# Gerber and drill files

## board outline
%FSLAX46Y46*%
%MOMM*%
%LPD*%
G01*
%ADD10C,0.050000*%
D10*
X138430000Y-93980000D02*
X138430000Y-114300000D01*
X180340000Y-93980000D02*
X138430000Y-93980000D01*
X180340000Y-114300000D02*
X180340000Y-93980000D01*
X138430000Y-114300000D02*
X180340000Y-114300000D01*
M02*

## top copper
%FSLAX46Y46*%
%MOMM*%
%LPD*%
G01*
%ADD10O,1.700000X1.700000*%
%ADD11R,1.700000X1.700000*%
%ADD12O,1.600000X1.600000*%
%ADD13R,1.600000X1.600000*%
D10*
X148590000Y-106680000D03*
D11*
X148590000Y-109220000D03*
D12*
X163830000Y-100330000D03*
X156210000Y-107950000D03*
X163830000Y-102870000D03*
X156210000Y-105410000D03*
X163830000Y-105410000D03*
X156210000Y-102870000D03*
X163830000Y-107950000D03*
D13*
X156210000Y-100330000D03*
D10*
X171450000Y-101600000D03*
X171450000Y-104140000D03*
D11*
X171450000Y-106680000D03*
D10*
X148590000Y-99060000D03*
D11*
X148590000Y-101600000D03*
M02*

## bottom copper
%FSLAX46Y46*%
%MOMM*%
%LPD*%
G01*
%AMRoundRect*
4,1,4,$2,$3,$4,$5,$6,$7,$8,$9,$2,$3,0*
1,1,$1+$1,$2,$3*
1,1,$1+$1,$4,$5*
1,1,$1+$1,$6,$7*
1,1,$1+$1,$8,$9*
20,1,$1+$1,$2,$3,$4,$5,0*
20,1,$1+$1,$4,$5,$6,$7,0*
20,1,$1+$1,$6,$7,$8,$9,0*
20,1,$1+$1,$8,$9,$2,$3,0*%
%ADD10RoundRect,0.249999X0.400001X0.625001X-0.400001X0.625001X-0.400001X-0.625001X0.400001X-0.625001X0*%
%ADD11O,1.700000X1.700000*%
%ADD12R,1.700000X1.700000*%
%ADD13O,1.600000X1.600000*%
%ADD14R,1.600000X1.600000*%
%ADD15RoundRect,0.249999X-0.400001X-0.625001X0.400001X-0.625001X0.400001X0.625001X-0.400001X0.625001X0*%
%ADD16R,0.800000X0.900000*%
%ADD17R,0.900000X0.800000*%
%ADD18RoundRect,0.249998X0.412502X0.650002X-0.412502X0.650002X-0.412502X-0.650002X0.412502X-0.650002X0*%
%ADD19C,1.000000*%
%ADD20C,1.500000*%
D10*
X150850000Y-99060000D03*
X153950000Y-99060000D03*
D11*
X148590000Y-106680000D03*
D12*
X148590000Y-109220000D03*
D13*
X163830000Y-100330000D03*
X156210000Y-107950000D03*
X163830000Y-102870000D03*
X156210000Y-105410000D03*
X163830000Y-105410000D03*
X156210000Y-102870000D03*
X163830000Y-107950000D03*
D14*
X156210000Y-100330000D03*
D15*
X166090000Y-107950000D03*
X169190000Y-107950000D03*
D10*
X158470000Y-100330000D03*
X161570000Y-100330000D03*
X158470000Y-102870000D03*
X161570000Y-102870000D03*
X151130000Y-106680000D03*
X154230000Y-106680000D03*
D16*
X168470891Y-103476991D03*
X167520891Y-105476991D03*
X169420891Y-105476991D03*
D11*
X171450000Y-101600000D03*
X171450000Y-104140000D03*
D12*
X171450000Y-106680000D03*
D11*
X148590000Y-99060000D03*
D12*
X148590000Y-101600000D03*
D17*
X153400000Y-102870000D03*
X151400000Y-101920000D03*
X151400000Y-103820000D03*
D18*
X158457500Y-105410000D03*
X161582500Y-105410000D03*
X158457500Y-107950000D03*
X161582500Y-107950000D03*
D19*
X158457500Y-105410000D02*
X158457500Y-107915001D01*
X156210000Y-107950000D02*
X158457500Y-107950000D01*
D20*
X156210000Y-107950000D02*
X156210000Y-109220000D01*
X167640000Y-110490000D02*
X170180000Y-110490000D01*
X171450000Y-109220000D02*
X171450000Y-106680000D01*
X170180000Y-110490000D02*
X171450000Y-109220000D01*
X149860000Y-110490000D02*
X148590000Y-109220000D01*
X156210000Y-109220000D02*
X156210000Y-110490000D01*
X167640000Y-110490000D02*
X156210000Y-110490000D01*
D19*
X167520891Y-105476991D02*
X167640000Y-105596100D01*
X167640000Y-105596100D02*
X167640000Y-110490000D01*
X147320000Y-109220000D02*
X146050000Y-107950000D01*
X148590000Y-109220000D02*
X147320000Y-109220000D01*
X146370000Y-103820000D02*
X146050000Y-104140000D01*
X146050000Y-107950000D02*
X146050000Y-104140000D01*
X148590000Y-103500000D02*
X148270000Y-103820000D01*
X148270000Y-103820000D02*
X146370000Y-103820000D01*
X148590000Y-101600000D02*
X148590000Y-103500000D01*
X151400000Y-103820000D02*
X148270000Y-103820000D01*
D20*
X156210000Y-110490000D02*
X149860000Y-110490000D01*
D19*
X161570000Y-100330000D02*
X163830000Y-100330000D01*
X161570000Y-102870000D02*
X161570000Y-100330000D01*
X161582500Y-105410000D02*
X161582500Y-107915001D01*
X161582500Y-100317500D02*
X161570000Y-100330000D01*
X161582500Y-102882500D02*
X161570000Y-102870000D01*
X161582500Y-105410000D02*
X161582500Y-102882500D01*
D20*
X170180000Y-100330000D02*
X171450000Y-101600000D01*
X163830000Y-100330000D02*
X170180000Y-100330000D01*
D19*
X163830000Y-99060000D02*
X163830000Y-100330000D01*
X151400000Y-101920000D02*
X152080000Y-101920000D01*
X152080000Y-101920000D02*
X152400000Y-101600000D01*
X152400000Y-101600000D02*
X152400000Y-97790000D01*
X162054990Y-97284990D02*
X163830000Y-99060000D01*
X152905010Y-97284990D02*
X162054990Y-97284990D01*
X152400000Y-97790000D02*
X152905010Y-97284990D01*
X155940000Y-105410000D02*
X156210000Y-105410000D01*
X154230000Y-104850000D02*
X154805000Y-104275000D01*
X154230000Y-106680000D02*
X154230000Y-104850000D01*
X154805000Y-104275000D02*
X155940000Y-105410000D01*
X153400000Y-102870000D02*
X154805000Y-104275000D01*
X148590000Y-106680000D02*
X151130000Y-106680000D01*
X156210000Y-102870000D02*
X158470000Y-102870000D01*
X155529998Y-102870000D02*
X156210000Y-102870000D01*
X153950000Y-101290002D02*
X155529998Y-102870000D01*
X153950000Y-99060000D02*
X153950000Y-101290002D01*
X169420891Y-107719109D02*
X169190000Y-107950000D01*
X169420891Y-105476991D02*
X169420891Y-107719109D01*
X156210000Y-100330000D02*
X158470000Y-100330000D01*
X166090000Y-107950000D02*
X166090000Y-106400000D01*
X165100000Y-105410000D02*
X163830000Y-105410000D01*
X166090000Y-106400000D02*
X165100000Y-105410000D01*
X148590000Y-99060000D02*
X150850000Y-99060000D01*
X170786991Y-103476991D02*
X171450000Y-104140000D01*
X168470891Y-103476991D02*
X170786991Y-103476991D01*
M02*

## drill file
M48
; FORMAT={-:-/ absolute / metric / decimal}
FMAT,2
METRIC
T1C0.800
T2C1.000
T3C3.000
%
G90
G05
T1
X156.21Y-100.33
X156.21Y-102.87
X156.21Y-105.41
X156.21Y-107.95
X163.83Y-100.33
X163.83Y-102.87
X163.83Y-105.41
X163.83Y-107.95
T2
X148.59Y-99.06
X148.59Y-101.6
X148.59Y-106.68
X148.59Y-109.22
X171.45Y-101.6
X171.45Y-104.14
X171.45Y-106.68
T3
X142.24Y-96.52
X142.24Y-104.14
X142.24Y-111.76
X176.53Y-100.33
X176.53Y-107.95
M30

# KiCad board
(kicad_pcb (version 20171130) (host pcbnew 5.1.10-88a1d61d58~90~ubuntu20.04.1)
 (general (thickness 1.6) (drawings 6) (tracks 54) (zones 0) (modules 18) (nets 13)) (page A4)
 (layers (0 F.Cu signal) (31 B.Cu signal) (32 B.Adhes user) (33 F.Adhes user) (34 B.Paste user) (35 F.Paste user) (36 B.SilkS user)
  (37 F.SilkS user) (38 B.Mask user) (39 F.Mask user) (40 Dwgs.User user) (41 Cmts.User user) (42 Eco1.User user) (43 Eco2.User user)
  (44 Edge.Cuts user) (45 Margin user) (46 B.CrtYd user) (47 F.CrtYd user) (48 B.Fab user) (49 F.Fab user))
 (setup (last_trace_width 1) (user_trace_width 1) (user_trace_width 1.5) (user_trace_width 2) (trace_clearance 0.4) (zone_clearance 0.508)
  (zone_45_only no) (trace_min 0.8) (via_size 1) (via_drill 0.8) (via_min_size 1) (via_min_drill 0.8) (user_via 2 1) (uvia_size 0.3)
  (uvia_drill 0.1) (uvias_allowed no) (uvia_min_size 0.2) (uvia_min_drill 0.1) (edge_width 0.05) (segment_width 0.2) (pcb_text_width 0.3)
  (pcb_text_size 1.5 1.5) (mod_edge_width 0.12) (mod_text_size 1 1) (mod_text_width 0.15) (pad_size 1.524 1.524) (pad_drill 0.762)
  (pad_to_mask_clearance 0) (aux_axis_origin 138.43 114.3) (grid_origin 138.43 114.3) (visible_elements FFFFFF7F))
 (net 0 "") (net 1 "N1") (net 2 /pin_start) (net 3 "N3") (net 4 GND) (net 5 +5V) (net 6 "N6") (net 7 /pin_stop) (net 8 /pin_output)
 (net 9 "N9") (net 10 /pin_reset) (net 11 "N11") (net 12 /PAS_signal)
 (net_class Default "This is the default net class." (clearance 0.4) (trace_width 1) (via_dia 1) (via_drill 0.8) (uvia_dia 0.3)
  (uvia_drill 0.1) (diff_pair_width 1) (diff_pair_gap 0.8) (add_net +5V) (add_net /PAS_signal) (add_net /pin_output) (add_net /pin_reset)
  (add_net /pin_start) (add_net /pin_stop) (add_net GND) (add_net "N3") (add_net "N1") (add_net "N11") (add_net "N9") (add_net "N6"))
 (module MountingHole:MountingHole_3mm (layer F.Cu) (at 176.53 107.95)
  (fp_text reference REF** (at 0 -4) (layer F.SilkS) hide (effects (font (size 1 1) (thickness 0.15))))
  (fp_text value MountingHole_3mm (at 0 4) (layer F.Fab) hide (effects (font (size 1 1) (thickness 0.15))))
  (pad 1 np_thru_hole circle (at 0 0) (size 3 3) (drill 3) (layers *.Cu *.Mask)))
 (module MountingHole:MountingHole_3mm (layer F.Cu) (at 176.53 100.33)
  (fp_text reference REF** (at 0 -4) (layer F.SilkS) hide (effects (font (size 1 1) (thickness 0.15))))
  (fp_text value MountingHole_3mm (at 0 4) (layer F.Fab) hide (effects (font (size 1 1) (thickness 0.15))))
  (pad 1 np_thru_hole circle (at 0 0) (size 3 3) (drill 3) (layers *.Cu *.Mask)))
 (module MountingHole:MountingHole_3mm (layer F.Cu) (at 142.24 104.14)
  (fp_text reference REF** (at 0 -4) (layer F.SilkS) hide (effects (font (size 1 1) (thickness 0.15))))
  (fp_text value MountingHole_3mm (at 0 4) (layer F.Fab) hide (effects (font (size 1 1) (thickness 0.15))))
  (pad 1 np_thru_hole circle (at 0 0) (size 3 3) (drill 3) (layers *.Cu *.Mask)))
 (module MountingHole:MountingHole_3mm (layer F.Cu) (at 142.24 111.76)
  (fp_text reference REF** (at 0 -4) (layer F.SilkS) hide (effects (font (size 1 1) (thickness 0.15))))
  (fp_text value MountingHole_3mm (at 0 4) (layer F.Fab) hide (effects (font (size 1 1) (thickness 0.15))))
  (pad 1 np_thru_hole circle (at 0 0) (size 3 3) (drill 3) (layers *.Cu *.Mask)))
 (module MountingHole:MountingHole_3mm (layer F.Cu) (at 142.24 96.52)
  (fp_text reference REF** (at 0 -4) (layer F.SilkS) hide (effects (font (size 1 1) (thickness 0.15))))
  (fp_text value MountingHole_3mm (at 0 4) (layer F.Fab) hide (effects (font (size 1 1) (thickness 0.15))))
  (pad 1 np_thru_hole circle (at 0 0) (size 3 3) (drill 3) (layers *.Cu *.Mask)))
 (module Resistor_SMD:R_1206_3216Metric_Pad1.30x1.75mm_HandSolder (layer B.Cu) (at 152.4 99.06 180)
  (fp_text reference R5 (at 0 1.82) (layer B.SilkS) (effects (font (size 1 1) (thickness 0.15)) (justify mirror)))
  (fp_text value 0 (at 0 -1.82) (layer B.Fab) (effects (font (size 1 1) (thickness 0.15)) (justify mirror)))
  (pad 2 smd roundrect (at 1.55 0 180) (size 1.3 1.75) (layers B.Cu B.Paste B.Mask) (roundrect_rratio 0.1923069230769231) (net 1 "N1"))
  (pad 1 smd roundrect (at -1.55 0 180) (size 1.3 1.75) (layers B.Cu B.Paste B.Mask) (roundrect_rratio 0.1923069230769231)
   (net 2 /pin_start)))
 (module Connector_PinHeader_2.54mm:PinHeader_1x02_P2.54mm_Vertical (layer F.Cu) (at 148.59 109.22 180)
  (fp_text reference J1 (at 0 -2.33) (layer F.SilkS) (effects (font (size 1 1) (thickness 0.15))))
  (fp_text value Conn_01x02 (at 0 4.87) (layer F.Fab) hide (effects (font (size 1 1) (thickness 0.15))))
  (pad 2 thru_hole oval (at 0 2.54 180) (size 1.7 1.7) (drill 1) (layers *.Cu *.Mask) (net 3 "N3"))
  (pad 1 thru_hole rect (at 0 0 180) (size 1.7 1.7) (drill 1) (layers *.Cu *.Mask) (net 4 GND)))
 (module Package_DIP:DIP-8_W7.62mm (layer F.Cu) (at 156.21 100.33)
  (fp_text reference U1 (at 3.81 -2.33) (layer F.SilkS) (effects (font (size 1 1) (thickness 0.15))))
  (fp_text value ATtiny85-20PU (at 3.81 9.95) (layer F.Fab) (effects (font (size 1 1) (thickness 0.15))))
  (pad 8 thru_hole oval (at 7.62 0) (size 1.6 1.6) (drill 0.8) (layers *.Cu *.Mask) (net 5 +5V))
  (pad 4 thru_hole oval (at 0 7.62) (size 1.6 1.6) (drill 0.8) (layers *.Cu *.Mask) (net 4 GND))
  (pad 7 thru_hole oval (at 7.62 2.54) (size 1.6 1.6) (drill 0.8) (layers *.Cu *.Mask) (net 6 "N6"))
  (pad 3 thru_hole oval (at 0 5.08) (size 1.6 1.6) (drill 0.8) (layers *.Cu *.Mask) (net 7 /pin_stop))
  (pad 6 thru_hole oval (at 7.62 5.08) (size 1.6 1.6) (drill 0.8) (layers *.Cu *.Mask) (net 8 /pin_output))
  (pad 2 thru_hole oval (at 0 2.54) (size 1.6 1.6) (drill 0.8) (layers *.Cu *.Mask) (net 2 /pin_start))
  (pad 5 thru_hole oval (at 7.62 7.62) (size 1.6 1.6) (drill 0.8) (layers *.Cu *.Mask) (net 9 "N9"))
  (pad 1 thru_hole rect (at 0 0) (size 1.6 1.6) (drill 0.8) (layers *.Cu *.Mask) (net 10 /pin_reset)))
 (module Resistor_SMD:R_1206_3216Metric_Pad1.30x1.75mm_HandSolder (layer B.Cu) (at 167.64 107.95)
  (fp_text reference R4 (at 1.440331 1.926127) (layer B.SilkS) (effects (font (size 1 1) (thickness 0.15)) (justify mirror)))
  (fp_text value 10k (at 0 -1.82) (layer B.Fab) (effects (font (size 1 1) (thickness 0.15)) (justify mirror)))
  (pad 1 smd roundrect (at -1.55 0) (size 1.3 1.75) (layers B.Cu B.Paste B.Mask) (roundrect_rratio 0.1923069230769231) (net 8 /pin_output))
  (pad 2 smd roundrect (at 1.55 0) (size 1.3 1.75) (layers B.Cu B.Paste B.Mask) (roundrect_rratio 0.1923069230769231) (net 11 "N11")))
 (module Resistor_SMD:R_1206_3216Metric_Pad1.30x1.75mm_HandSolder (layer B.Cu) (at 160.02 100.33 180)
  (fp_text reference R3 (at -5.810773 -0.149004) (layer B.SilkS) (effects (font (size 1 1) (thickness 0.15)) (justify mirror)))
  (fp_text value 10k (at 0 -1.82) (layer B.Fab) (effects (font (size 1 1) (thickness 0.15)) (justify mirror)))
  (pad 2 smd roundrect (at 1.55 0 180) (size 1.3 1.75) (layers B.Cu B.Paste B.Mask) (roundrect_rratio 0.1923069230769231)
   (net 10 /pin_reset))
  (pad 1 smd roundrect (at -1.55 0 180) (size 1.3 1.75) (layers B.Cu B.Paste B.Mask) (roundrect_rratio 0.1923069230769231) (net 5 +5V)))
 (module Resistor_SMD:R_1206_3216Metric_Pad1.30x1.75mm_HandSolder (layer B.Cu) (at 160.02 102.87 180)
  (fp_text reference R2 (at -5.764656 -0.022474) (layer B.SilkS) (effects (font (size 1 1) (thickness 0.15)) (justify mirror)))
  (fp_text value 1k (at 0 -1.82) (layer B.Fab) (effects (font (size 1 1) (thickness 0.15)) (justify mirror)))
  (pad 2 smd roundrect (at 1.55 0 180) (size 1.3 1.75) (layers B.Cu B.Paste B.Mask) (roundrect_rratio 0.1923069230769231) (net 2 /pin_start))
  (pad 1 smd roundrect (at -1.55 0 180) (size 1.3 1.75) (layers B.Cu B.Paste B.Mask) (roundrect_rratio 0.1923069230769231) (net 5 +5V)))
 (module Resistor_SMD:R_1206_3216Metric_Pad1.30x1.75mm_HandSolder (layer B.Cu) (at 152.68 106.68 180)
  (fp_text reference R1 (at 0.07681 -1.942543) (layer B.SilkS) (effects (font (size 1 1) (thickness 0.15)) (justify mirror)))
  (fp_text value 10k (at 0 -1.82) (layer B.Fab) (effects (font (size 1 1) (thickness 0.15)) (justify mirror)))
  (pad 2 smd roundrect (at 1.55 0 180) (size 1.3 1.75) (layers B.Cu B.Paste B.Mask) (roundrect_rratio 0.1923069230769231) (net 3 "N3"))
  (pad 1 smd roundrect (at -1.55 0 180) (size 1.3 1.75) (layers B.Cu B.Paste B.Mask) (roundrect_rratio 0.1923069230769231) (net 7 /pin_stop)))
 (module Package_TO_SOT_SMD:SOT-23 (layer B.Cu) (at 168.470891 104.476991 90)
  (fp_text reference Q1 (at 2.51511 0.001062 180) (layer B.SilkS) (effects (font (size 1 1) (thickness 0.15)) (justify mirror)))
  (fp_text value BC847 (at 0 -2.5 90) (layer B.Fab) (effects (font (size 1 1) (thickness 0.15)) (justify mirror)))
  (pad 3 smd rect (at 1 0 90) (size 0.9 0.8) (layers B.Cu B.Paste B.Mask) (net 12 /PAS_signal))
  (pad 2 smd rect (at -1 -0.95 90) (size 0.9 0.8) (layers B.Cu B.Paste B.Mask) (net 4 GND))
  (pad 1 smd rect (at -1 0.95 90) (size 0.9 0.8) (layers B.Cu B.Paste B.Mask) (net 11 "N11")))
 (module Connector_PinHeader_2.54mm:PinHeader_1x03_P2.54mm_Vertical (layer F.Cu) (at 171.45 106.68 180)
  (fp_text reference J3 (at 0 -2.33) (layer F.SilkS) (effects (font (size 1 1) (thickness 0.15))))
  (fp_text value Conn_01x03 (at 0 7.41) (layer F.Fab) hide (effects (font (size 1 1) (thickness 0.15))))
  (pad 3 thru_hole oval (at 0 5.08 180) (size 1.7 1.7) (drill 1) (layers *.Cu *.Mask) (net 5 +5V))
  (pad 2 thru_hole oval (at 0 2.54 180) (size 1.7 1.7) (drill 1) (layers *.Cu *.Mask) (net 12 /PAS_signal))
  (pad 1 thru_hole rect (at 0 0 180) (size 1.7 1.7) (drill 1) (layers *.Cu *.Mask) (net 4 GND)))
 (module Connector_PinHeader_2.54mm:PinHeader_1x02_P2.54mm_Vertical (layer F.Cu) (at 148.59 101.6 180)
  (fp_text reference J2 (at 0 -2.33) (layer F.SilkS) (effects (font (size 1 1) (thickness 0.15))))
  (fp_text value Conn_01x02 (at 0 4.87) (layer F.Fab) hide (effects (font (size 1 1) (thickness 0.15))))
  (pad 2 thru_hole oval (at 0 2.54 180) (size 1.7 1.7) (drill 1) (layers *.Cu *.Mask) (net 1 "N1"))
  (pad 1 thru_hole rect (at 0 0 180) (size 1.7 1.7) (drill 1) (layers *.Cu *.Mask) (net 4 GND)))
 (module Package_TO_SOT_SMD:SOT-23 (layer B.Cu) (at 152.4 102.87)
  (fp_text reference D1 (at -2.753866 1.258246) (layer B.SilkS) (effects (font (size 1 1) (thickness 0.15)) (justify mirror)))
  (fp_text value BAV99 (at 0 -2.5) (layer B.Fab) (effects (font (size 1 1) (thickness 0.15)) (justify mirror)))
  (pad 3 smd rect (at 1 0) (size 0.9 0.8) (layers B.Cu B.Paste B.Mask) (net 7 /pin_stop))
  (pad 2 smd rect (at -1 -0.95) (size 0.9 0.8) (layers B.Cu B.Paste B.Mask) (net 5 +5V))
  (pad 1 smd rect (at -1 0.95) (size 0.9 0.8) (layers B.Cu B.Paste B.Mask) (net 4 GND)))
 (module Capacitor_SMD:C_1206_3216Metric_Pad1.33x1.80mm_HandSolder (layer B.Cu) (at 160.02 105.41 180)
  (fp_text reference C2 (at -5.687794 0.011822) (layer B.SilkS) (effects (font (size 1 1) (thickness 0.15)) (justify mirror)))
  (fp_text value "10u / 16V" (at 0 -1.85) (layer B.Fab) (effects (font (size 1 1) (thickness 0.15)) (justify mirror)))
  (pad 2 smd roundrect (at 1.5625 0 180) (size 1.325 1.8) (layers B.Cu B.Paste B.Mask) (roundrect_rratio 0.1886777358490566) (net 4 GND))
  (pad 1 smd roundrect (at -1.5625 0 180) (size 1.325 1.8) (layers B.Cu B.Paste B.Mask) (roundrect_rratio 0.1886777358490566) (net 5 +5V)))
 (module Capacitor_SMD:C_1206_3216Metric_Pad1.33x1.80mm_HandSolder (layer B.Cu) (at 160.02 107.95 180)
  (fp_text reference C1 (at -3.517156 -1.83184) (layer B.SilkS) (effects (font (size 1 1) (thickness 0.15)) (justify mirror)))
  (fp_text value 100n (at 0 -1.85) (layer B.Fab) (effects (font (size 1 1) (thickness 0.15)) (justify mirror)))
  (pad 2 smd roundrect (at 1.5625 0 180) (size 1.325 1.8) (layers B.Cu B.Paste B.Mask) (roundrect_rratio 0.1886777358490566) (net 4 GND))
  (pad 1 smd roundrect (at -1.5625 0 180) (size 1.325 1.8) (layers B.Cu B.Paste B.Mask) (roundrect_rratio 0.1886777358490566) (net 5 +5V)))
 (gr_line (start 138.43 93.98) (end 138.43 114.3) (layer Edge.Cuts) (width 0.05))
 (gr_line (start 180.34 93.98) (end 138.43 93.98) (layer Edge.Cuts) (width 0.05))
 (gr_line (start 180.34 114.3) (end 180.34 93.98) (layer Edge.Cuts) (width 0.05))
 (gr_line (start 138.43 114.3) (end 180.34 114.3) (layer Edge.Cuts) (width 0.05))
 (segment (start 158.4575 105.41) (end 158.4575 107.915001) (width 1) (layer B.Cu) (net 4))
 (segment (start 156.21 107.95) (end 158.4575 107.95) (width 1) (layer B.Cu) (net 4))
 (segment (start 156.21 107.95) (end 156.21 109.22) (width 1.5) (layer B.Cu) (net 4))
 (segment (start 167.64 110.49) (end 170.18 110.49) (width 1.5) (layer B.Cu) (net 4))
 (segment (start 171.45 109.22) (end 171.45 106.68) (width 1.5) (layer B.Cu) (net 4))
 (segment (start 170.18 110.49) (end 171.45 109.22) (width 1.5) (layer B.Cu) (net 4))
 (segment (start 149.86 110.49) (end 148.59 109.22) (width 1.5) (layer B.Cu) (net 4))
 (segment (start 156.21 109.22) (end 156.21 110.49) (width 1.5) (layer B.Cu) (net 4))
 (segment (start 167.64 110.49) (end 156.21 110.49) (width 1.5) (layer B.Cu) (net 4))
 (segment (start 167.520891 105.476991) (end 167.64 105.5961) (width 1) (layer B.Cu) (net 4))
 (segment (start 167.64 105.5961) (end 167.64 110.49) (width 1) (layer B.Cu) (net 4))
 (segment (start 147.32 109.22) (end 146.05 107.95) (width 1) (layer B.Cu) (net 4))
 (segment (start 148.59 109.22) (end 147.32 109.22) (width 1) (layer B.Cu) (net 4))
 (segment (start 146.37 103.82) (end 146.05 104.14) (width 1) (layer B.Cu) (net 4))
 (segment (start 146.05 107.95) (end 146.05 104.14) (width 1) (layer B.Cu) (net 4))
 (segment (start 148.59 103.5) (end 148.27 103.82) (width 1) (layer B.Cu) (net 4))
 (segment (start 148.27 103.82) (end 146.37 103.82) (width 1) (layer B.Cu) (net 4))
 (segment (start 148.59 101.6) (end 148.59 103.5) (width 1) (layer B.Cu) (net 4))
 (segment (start 151.4 103.82) (end 148.27 103.82) (width 1) (layer B.Cu) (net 4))
 (segment (start 156.21 110.49) (end 149.86 110.49) (width 1.5) (layer B.Cu) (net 4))
 (segment (start 161.57 100.33) (end 163.83 100.33) (width 1) (layer B.Cu) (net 5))
 (segment (start 161.57 102.87) (end 161.57 100.33) (width 1) (layer B.Cu) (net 5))
 (segment (start 161.5825 105.41) (end 161.5825 107.915001) (width 1) (layer B.Cu) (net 5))
 (segment (start 161.5825 100.3175) (end 161.57 100.33) (width 1) (layer B.Cu) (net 5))
 (segment (start 161.5825 102.8825) (end 161.57 102.87) (width 1) (layer B.Cu) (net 5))
 (segment (start 161.5825 105.41) (end 161.5825 102.8825) (width 1) (layer B.Cu) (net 5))
 (segment (start 170.18 100.33) (end 171.45 101.6) (width 1.5) (layer B.Cu) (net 5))
 (segment (start 163.83 100.33) (end 170.18 100.33) (width 1.5) (layer B.Cu) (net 5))
 (segment (start 163.83 99.06) (end 163.83 100.33) (width 1) (layer B.Cu) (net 5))
 (segment (start 151.4 101.92) (end 152.08 101.92) (width 1) (layer B.Cu) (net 5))
 (segment (start 152.08 101.92) (end 152.4 101.6) (width 1) (layer B.Cu) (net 5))
 (segment (start 152.4 101.6) (end 152.4 97.79) (width 1) (layer B.Cu) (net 5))
 (segment (start 162.05499 97.28499) (end 163.83 99.06) (width 1) (layer B.Cu) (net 5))
 (segment (start 152.90501 97.28499) (end 162.05499 97.28499) (width 1) (layer B.Cu) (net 5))
 (segment (start 152.4 97.79) (end 152.90501 97.28499) (width 1) (layer B.Cu) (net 5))
 (segment (start 155.94 105.41) (end 156.21 105.41) (width 1) (layer B.Cu) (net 7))
 (segment (start 154.23 104.85) (end 154.805 104.275) (width 1) (layer B.Cu) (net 7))
 (segment (start 154.23 106.68) (end 154.23 104.85) (width 1) (layer B.Cu) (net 7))
 (segment (start 154.805 104.275) (end 155.94 105.41) (width 1) (layer B.Cu) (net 7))
 (segment (start 153.4 102.87) (end 154.805 104.275) (width 1) (layer B.Cu) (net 7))
 (segment (start 148.59 106.68) (end 151.13 106.68) (width 1) (layer B.Cu) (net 3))
 (segment (start 156.21 102.87) (end 158.47 102.87) (width 1) (layer B.Cu) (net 2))
 (segment (start 155.529998 102.87) (end 156.21 102.87) (width 1) (layer B.Cu) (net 2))
 (segment (start 153.95 101.290002) (end 155.529998 102.87) (width 1) (layer B.Cu) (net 2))
 (segment (start 153.95 99.06) (end 153.95 101.290002) (width 1) (layer B.Cu) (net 2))
 (segment (start 169.420891 107.719109) (end 169.19 107.95) (width 1) (layer B.Cu) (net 11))
 (segment (start 169.420891 105.476991) (end 169.420891 107.719109) (width 1) (layer B.Cu) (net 11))
 (segment (start 156.21 100.33) (end 158.47 100.33) (width 1) (layer B.Cu) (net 10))
 (segment (start 166.09 107.95) (end 166.09 106.4) (width 1) (layer B.Cu) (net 8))
 (segment (start 165.1 105.41) (end 163.83 105.41) (width 1) (layer B.Cu) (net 8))
 (segment (start 166.09 106.4) (end 165.1 105.41) (width 1) (layer B.Cu) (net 8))
 (segment (start 148.59 99.06) (end 150.85 99.06) (width 1) (layer B.Cu) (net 1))
 (segment (start 170.786991 103.476991) (end 171.45 104.14) (width 1) (layer B.Cu) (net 12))
 (segment (start 168.470891 103.476991) (end 170.786991 103.476991) (width 1) (layer B.Cu) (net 12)))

